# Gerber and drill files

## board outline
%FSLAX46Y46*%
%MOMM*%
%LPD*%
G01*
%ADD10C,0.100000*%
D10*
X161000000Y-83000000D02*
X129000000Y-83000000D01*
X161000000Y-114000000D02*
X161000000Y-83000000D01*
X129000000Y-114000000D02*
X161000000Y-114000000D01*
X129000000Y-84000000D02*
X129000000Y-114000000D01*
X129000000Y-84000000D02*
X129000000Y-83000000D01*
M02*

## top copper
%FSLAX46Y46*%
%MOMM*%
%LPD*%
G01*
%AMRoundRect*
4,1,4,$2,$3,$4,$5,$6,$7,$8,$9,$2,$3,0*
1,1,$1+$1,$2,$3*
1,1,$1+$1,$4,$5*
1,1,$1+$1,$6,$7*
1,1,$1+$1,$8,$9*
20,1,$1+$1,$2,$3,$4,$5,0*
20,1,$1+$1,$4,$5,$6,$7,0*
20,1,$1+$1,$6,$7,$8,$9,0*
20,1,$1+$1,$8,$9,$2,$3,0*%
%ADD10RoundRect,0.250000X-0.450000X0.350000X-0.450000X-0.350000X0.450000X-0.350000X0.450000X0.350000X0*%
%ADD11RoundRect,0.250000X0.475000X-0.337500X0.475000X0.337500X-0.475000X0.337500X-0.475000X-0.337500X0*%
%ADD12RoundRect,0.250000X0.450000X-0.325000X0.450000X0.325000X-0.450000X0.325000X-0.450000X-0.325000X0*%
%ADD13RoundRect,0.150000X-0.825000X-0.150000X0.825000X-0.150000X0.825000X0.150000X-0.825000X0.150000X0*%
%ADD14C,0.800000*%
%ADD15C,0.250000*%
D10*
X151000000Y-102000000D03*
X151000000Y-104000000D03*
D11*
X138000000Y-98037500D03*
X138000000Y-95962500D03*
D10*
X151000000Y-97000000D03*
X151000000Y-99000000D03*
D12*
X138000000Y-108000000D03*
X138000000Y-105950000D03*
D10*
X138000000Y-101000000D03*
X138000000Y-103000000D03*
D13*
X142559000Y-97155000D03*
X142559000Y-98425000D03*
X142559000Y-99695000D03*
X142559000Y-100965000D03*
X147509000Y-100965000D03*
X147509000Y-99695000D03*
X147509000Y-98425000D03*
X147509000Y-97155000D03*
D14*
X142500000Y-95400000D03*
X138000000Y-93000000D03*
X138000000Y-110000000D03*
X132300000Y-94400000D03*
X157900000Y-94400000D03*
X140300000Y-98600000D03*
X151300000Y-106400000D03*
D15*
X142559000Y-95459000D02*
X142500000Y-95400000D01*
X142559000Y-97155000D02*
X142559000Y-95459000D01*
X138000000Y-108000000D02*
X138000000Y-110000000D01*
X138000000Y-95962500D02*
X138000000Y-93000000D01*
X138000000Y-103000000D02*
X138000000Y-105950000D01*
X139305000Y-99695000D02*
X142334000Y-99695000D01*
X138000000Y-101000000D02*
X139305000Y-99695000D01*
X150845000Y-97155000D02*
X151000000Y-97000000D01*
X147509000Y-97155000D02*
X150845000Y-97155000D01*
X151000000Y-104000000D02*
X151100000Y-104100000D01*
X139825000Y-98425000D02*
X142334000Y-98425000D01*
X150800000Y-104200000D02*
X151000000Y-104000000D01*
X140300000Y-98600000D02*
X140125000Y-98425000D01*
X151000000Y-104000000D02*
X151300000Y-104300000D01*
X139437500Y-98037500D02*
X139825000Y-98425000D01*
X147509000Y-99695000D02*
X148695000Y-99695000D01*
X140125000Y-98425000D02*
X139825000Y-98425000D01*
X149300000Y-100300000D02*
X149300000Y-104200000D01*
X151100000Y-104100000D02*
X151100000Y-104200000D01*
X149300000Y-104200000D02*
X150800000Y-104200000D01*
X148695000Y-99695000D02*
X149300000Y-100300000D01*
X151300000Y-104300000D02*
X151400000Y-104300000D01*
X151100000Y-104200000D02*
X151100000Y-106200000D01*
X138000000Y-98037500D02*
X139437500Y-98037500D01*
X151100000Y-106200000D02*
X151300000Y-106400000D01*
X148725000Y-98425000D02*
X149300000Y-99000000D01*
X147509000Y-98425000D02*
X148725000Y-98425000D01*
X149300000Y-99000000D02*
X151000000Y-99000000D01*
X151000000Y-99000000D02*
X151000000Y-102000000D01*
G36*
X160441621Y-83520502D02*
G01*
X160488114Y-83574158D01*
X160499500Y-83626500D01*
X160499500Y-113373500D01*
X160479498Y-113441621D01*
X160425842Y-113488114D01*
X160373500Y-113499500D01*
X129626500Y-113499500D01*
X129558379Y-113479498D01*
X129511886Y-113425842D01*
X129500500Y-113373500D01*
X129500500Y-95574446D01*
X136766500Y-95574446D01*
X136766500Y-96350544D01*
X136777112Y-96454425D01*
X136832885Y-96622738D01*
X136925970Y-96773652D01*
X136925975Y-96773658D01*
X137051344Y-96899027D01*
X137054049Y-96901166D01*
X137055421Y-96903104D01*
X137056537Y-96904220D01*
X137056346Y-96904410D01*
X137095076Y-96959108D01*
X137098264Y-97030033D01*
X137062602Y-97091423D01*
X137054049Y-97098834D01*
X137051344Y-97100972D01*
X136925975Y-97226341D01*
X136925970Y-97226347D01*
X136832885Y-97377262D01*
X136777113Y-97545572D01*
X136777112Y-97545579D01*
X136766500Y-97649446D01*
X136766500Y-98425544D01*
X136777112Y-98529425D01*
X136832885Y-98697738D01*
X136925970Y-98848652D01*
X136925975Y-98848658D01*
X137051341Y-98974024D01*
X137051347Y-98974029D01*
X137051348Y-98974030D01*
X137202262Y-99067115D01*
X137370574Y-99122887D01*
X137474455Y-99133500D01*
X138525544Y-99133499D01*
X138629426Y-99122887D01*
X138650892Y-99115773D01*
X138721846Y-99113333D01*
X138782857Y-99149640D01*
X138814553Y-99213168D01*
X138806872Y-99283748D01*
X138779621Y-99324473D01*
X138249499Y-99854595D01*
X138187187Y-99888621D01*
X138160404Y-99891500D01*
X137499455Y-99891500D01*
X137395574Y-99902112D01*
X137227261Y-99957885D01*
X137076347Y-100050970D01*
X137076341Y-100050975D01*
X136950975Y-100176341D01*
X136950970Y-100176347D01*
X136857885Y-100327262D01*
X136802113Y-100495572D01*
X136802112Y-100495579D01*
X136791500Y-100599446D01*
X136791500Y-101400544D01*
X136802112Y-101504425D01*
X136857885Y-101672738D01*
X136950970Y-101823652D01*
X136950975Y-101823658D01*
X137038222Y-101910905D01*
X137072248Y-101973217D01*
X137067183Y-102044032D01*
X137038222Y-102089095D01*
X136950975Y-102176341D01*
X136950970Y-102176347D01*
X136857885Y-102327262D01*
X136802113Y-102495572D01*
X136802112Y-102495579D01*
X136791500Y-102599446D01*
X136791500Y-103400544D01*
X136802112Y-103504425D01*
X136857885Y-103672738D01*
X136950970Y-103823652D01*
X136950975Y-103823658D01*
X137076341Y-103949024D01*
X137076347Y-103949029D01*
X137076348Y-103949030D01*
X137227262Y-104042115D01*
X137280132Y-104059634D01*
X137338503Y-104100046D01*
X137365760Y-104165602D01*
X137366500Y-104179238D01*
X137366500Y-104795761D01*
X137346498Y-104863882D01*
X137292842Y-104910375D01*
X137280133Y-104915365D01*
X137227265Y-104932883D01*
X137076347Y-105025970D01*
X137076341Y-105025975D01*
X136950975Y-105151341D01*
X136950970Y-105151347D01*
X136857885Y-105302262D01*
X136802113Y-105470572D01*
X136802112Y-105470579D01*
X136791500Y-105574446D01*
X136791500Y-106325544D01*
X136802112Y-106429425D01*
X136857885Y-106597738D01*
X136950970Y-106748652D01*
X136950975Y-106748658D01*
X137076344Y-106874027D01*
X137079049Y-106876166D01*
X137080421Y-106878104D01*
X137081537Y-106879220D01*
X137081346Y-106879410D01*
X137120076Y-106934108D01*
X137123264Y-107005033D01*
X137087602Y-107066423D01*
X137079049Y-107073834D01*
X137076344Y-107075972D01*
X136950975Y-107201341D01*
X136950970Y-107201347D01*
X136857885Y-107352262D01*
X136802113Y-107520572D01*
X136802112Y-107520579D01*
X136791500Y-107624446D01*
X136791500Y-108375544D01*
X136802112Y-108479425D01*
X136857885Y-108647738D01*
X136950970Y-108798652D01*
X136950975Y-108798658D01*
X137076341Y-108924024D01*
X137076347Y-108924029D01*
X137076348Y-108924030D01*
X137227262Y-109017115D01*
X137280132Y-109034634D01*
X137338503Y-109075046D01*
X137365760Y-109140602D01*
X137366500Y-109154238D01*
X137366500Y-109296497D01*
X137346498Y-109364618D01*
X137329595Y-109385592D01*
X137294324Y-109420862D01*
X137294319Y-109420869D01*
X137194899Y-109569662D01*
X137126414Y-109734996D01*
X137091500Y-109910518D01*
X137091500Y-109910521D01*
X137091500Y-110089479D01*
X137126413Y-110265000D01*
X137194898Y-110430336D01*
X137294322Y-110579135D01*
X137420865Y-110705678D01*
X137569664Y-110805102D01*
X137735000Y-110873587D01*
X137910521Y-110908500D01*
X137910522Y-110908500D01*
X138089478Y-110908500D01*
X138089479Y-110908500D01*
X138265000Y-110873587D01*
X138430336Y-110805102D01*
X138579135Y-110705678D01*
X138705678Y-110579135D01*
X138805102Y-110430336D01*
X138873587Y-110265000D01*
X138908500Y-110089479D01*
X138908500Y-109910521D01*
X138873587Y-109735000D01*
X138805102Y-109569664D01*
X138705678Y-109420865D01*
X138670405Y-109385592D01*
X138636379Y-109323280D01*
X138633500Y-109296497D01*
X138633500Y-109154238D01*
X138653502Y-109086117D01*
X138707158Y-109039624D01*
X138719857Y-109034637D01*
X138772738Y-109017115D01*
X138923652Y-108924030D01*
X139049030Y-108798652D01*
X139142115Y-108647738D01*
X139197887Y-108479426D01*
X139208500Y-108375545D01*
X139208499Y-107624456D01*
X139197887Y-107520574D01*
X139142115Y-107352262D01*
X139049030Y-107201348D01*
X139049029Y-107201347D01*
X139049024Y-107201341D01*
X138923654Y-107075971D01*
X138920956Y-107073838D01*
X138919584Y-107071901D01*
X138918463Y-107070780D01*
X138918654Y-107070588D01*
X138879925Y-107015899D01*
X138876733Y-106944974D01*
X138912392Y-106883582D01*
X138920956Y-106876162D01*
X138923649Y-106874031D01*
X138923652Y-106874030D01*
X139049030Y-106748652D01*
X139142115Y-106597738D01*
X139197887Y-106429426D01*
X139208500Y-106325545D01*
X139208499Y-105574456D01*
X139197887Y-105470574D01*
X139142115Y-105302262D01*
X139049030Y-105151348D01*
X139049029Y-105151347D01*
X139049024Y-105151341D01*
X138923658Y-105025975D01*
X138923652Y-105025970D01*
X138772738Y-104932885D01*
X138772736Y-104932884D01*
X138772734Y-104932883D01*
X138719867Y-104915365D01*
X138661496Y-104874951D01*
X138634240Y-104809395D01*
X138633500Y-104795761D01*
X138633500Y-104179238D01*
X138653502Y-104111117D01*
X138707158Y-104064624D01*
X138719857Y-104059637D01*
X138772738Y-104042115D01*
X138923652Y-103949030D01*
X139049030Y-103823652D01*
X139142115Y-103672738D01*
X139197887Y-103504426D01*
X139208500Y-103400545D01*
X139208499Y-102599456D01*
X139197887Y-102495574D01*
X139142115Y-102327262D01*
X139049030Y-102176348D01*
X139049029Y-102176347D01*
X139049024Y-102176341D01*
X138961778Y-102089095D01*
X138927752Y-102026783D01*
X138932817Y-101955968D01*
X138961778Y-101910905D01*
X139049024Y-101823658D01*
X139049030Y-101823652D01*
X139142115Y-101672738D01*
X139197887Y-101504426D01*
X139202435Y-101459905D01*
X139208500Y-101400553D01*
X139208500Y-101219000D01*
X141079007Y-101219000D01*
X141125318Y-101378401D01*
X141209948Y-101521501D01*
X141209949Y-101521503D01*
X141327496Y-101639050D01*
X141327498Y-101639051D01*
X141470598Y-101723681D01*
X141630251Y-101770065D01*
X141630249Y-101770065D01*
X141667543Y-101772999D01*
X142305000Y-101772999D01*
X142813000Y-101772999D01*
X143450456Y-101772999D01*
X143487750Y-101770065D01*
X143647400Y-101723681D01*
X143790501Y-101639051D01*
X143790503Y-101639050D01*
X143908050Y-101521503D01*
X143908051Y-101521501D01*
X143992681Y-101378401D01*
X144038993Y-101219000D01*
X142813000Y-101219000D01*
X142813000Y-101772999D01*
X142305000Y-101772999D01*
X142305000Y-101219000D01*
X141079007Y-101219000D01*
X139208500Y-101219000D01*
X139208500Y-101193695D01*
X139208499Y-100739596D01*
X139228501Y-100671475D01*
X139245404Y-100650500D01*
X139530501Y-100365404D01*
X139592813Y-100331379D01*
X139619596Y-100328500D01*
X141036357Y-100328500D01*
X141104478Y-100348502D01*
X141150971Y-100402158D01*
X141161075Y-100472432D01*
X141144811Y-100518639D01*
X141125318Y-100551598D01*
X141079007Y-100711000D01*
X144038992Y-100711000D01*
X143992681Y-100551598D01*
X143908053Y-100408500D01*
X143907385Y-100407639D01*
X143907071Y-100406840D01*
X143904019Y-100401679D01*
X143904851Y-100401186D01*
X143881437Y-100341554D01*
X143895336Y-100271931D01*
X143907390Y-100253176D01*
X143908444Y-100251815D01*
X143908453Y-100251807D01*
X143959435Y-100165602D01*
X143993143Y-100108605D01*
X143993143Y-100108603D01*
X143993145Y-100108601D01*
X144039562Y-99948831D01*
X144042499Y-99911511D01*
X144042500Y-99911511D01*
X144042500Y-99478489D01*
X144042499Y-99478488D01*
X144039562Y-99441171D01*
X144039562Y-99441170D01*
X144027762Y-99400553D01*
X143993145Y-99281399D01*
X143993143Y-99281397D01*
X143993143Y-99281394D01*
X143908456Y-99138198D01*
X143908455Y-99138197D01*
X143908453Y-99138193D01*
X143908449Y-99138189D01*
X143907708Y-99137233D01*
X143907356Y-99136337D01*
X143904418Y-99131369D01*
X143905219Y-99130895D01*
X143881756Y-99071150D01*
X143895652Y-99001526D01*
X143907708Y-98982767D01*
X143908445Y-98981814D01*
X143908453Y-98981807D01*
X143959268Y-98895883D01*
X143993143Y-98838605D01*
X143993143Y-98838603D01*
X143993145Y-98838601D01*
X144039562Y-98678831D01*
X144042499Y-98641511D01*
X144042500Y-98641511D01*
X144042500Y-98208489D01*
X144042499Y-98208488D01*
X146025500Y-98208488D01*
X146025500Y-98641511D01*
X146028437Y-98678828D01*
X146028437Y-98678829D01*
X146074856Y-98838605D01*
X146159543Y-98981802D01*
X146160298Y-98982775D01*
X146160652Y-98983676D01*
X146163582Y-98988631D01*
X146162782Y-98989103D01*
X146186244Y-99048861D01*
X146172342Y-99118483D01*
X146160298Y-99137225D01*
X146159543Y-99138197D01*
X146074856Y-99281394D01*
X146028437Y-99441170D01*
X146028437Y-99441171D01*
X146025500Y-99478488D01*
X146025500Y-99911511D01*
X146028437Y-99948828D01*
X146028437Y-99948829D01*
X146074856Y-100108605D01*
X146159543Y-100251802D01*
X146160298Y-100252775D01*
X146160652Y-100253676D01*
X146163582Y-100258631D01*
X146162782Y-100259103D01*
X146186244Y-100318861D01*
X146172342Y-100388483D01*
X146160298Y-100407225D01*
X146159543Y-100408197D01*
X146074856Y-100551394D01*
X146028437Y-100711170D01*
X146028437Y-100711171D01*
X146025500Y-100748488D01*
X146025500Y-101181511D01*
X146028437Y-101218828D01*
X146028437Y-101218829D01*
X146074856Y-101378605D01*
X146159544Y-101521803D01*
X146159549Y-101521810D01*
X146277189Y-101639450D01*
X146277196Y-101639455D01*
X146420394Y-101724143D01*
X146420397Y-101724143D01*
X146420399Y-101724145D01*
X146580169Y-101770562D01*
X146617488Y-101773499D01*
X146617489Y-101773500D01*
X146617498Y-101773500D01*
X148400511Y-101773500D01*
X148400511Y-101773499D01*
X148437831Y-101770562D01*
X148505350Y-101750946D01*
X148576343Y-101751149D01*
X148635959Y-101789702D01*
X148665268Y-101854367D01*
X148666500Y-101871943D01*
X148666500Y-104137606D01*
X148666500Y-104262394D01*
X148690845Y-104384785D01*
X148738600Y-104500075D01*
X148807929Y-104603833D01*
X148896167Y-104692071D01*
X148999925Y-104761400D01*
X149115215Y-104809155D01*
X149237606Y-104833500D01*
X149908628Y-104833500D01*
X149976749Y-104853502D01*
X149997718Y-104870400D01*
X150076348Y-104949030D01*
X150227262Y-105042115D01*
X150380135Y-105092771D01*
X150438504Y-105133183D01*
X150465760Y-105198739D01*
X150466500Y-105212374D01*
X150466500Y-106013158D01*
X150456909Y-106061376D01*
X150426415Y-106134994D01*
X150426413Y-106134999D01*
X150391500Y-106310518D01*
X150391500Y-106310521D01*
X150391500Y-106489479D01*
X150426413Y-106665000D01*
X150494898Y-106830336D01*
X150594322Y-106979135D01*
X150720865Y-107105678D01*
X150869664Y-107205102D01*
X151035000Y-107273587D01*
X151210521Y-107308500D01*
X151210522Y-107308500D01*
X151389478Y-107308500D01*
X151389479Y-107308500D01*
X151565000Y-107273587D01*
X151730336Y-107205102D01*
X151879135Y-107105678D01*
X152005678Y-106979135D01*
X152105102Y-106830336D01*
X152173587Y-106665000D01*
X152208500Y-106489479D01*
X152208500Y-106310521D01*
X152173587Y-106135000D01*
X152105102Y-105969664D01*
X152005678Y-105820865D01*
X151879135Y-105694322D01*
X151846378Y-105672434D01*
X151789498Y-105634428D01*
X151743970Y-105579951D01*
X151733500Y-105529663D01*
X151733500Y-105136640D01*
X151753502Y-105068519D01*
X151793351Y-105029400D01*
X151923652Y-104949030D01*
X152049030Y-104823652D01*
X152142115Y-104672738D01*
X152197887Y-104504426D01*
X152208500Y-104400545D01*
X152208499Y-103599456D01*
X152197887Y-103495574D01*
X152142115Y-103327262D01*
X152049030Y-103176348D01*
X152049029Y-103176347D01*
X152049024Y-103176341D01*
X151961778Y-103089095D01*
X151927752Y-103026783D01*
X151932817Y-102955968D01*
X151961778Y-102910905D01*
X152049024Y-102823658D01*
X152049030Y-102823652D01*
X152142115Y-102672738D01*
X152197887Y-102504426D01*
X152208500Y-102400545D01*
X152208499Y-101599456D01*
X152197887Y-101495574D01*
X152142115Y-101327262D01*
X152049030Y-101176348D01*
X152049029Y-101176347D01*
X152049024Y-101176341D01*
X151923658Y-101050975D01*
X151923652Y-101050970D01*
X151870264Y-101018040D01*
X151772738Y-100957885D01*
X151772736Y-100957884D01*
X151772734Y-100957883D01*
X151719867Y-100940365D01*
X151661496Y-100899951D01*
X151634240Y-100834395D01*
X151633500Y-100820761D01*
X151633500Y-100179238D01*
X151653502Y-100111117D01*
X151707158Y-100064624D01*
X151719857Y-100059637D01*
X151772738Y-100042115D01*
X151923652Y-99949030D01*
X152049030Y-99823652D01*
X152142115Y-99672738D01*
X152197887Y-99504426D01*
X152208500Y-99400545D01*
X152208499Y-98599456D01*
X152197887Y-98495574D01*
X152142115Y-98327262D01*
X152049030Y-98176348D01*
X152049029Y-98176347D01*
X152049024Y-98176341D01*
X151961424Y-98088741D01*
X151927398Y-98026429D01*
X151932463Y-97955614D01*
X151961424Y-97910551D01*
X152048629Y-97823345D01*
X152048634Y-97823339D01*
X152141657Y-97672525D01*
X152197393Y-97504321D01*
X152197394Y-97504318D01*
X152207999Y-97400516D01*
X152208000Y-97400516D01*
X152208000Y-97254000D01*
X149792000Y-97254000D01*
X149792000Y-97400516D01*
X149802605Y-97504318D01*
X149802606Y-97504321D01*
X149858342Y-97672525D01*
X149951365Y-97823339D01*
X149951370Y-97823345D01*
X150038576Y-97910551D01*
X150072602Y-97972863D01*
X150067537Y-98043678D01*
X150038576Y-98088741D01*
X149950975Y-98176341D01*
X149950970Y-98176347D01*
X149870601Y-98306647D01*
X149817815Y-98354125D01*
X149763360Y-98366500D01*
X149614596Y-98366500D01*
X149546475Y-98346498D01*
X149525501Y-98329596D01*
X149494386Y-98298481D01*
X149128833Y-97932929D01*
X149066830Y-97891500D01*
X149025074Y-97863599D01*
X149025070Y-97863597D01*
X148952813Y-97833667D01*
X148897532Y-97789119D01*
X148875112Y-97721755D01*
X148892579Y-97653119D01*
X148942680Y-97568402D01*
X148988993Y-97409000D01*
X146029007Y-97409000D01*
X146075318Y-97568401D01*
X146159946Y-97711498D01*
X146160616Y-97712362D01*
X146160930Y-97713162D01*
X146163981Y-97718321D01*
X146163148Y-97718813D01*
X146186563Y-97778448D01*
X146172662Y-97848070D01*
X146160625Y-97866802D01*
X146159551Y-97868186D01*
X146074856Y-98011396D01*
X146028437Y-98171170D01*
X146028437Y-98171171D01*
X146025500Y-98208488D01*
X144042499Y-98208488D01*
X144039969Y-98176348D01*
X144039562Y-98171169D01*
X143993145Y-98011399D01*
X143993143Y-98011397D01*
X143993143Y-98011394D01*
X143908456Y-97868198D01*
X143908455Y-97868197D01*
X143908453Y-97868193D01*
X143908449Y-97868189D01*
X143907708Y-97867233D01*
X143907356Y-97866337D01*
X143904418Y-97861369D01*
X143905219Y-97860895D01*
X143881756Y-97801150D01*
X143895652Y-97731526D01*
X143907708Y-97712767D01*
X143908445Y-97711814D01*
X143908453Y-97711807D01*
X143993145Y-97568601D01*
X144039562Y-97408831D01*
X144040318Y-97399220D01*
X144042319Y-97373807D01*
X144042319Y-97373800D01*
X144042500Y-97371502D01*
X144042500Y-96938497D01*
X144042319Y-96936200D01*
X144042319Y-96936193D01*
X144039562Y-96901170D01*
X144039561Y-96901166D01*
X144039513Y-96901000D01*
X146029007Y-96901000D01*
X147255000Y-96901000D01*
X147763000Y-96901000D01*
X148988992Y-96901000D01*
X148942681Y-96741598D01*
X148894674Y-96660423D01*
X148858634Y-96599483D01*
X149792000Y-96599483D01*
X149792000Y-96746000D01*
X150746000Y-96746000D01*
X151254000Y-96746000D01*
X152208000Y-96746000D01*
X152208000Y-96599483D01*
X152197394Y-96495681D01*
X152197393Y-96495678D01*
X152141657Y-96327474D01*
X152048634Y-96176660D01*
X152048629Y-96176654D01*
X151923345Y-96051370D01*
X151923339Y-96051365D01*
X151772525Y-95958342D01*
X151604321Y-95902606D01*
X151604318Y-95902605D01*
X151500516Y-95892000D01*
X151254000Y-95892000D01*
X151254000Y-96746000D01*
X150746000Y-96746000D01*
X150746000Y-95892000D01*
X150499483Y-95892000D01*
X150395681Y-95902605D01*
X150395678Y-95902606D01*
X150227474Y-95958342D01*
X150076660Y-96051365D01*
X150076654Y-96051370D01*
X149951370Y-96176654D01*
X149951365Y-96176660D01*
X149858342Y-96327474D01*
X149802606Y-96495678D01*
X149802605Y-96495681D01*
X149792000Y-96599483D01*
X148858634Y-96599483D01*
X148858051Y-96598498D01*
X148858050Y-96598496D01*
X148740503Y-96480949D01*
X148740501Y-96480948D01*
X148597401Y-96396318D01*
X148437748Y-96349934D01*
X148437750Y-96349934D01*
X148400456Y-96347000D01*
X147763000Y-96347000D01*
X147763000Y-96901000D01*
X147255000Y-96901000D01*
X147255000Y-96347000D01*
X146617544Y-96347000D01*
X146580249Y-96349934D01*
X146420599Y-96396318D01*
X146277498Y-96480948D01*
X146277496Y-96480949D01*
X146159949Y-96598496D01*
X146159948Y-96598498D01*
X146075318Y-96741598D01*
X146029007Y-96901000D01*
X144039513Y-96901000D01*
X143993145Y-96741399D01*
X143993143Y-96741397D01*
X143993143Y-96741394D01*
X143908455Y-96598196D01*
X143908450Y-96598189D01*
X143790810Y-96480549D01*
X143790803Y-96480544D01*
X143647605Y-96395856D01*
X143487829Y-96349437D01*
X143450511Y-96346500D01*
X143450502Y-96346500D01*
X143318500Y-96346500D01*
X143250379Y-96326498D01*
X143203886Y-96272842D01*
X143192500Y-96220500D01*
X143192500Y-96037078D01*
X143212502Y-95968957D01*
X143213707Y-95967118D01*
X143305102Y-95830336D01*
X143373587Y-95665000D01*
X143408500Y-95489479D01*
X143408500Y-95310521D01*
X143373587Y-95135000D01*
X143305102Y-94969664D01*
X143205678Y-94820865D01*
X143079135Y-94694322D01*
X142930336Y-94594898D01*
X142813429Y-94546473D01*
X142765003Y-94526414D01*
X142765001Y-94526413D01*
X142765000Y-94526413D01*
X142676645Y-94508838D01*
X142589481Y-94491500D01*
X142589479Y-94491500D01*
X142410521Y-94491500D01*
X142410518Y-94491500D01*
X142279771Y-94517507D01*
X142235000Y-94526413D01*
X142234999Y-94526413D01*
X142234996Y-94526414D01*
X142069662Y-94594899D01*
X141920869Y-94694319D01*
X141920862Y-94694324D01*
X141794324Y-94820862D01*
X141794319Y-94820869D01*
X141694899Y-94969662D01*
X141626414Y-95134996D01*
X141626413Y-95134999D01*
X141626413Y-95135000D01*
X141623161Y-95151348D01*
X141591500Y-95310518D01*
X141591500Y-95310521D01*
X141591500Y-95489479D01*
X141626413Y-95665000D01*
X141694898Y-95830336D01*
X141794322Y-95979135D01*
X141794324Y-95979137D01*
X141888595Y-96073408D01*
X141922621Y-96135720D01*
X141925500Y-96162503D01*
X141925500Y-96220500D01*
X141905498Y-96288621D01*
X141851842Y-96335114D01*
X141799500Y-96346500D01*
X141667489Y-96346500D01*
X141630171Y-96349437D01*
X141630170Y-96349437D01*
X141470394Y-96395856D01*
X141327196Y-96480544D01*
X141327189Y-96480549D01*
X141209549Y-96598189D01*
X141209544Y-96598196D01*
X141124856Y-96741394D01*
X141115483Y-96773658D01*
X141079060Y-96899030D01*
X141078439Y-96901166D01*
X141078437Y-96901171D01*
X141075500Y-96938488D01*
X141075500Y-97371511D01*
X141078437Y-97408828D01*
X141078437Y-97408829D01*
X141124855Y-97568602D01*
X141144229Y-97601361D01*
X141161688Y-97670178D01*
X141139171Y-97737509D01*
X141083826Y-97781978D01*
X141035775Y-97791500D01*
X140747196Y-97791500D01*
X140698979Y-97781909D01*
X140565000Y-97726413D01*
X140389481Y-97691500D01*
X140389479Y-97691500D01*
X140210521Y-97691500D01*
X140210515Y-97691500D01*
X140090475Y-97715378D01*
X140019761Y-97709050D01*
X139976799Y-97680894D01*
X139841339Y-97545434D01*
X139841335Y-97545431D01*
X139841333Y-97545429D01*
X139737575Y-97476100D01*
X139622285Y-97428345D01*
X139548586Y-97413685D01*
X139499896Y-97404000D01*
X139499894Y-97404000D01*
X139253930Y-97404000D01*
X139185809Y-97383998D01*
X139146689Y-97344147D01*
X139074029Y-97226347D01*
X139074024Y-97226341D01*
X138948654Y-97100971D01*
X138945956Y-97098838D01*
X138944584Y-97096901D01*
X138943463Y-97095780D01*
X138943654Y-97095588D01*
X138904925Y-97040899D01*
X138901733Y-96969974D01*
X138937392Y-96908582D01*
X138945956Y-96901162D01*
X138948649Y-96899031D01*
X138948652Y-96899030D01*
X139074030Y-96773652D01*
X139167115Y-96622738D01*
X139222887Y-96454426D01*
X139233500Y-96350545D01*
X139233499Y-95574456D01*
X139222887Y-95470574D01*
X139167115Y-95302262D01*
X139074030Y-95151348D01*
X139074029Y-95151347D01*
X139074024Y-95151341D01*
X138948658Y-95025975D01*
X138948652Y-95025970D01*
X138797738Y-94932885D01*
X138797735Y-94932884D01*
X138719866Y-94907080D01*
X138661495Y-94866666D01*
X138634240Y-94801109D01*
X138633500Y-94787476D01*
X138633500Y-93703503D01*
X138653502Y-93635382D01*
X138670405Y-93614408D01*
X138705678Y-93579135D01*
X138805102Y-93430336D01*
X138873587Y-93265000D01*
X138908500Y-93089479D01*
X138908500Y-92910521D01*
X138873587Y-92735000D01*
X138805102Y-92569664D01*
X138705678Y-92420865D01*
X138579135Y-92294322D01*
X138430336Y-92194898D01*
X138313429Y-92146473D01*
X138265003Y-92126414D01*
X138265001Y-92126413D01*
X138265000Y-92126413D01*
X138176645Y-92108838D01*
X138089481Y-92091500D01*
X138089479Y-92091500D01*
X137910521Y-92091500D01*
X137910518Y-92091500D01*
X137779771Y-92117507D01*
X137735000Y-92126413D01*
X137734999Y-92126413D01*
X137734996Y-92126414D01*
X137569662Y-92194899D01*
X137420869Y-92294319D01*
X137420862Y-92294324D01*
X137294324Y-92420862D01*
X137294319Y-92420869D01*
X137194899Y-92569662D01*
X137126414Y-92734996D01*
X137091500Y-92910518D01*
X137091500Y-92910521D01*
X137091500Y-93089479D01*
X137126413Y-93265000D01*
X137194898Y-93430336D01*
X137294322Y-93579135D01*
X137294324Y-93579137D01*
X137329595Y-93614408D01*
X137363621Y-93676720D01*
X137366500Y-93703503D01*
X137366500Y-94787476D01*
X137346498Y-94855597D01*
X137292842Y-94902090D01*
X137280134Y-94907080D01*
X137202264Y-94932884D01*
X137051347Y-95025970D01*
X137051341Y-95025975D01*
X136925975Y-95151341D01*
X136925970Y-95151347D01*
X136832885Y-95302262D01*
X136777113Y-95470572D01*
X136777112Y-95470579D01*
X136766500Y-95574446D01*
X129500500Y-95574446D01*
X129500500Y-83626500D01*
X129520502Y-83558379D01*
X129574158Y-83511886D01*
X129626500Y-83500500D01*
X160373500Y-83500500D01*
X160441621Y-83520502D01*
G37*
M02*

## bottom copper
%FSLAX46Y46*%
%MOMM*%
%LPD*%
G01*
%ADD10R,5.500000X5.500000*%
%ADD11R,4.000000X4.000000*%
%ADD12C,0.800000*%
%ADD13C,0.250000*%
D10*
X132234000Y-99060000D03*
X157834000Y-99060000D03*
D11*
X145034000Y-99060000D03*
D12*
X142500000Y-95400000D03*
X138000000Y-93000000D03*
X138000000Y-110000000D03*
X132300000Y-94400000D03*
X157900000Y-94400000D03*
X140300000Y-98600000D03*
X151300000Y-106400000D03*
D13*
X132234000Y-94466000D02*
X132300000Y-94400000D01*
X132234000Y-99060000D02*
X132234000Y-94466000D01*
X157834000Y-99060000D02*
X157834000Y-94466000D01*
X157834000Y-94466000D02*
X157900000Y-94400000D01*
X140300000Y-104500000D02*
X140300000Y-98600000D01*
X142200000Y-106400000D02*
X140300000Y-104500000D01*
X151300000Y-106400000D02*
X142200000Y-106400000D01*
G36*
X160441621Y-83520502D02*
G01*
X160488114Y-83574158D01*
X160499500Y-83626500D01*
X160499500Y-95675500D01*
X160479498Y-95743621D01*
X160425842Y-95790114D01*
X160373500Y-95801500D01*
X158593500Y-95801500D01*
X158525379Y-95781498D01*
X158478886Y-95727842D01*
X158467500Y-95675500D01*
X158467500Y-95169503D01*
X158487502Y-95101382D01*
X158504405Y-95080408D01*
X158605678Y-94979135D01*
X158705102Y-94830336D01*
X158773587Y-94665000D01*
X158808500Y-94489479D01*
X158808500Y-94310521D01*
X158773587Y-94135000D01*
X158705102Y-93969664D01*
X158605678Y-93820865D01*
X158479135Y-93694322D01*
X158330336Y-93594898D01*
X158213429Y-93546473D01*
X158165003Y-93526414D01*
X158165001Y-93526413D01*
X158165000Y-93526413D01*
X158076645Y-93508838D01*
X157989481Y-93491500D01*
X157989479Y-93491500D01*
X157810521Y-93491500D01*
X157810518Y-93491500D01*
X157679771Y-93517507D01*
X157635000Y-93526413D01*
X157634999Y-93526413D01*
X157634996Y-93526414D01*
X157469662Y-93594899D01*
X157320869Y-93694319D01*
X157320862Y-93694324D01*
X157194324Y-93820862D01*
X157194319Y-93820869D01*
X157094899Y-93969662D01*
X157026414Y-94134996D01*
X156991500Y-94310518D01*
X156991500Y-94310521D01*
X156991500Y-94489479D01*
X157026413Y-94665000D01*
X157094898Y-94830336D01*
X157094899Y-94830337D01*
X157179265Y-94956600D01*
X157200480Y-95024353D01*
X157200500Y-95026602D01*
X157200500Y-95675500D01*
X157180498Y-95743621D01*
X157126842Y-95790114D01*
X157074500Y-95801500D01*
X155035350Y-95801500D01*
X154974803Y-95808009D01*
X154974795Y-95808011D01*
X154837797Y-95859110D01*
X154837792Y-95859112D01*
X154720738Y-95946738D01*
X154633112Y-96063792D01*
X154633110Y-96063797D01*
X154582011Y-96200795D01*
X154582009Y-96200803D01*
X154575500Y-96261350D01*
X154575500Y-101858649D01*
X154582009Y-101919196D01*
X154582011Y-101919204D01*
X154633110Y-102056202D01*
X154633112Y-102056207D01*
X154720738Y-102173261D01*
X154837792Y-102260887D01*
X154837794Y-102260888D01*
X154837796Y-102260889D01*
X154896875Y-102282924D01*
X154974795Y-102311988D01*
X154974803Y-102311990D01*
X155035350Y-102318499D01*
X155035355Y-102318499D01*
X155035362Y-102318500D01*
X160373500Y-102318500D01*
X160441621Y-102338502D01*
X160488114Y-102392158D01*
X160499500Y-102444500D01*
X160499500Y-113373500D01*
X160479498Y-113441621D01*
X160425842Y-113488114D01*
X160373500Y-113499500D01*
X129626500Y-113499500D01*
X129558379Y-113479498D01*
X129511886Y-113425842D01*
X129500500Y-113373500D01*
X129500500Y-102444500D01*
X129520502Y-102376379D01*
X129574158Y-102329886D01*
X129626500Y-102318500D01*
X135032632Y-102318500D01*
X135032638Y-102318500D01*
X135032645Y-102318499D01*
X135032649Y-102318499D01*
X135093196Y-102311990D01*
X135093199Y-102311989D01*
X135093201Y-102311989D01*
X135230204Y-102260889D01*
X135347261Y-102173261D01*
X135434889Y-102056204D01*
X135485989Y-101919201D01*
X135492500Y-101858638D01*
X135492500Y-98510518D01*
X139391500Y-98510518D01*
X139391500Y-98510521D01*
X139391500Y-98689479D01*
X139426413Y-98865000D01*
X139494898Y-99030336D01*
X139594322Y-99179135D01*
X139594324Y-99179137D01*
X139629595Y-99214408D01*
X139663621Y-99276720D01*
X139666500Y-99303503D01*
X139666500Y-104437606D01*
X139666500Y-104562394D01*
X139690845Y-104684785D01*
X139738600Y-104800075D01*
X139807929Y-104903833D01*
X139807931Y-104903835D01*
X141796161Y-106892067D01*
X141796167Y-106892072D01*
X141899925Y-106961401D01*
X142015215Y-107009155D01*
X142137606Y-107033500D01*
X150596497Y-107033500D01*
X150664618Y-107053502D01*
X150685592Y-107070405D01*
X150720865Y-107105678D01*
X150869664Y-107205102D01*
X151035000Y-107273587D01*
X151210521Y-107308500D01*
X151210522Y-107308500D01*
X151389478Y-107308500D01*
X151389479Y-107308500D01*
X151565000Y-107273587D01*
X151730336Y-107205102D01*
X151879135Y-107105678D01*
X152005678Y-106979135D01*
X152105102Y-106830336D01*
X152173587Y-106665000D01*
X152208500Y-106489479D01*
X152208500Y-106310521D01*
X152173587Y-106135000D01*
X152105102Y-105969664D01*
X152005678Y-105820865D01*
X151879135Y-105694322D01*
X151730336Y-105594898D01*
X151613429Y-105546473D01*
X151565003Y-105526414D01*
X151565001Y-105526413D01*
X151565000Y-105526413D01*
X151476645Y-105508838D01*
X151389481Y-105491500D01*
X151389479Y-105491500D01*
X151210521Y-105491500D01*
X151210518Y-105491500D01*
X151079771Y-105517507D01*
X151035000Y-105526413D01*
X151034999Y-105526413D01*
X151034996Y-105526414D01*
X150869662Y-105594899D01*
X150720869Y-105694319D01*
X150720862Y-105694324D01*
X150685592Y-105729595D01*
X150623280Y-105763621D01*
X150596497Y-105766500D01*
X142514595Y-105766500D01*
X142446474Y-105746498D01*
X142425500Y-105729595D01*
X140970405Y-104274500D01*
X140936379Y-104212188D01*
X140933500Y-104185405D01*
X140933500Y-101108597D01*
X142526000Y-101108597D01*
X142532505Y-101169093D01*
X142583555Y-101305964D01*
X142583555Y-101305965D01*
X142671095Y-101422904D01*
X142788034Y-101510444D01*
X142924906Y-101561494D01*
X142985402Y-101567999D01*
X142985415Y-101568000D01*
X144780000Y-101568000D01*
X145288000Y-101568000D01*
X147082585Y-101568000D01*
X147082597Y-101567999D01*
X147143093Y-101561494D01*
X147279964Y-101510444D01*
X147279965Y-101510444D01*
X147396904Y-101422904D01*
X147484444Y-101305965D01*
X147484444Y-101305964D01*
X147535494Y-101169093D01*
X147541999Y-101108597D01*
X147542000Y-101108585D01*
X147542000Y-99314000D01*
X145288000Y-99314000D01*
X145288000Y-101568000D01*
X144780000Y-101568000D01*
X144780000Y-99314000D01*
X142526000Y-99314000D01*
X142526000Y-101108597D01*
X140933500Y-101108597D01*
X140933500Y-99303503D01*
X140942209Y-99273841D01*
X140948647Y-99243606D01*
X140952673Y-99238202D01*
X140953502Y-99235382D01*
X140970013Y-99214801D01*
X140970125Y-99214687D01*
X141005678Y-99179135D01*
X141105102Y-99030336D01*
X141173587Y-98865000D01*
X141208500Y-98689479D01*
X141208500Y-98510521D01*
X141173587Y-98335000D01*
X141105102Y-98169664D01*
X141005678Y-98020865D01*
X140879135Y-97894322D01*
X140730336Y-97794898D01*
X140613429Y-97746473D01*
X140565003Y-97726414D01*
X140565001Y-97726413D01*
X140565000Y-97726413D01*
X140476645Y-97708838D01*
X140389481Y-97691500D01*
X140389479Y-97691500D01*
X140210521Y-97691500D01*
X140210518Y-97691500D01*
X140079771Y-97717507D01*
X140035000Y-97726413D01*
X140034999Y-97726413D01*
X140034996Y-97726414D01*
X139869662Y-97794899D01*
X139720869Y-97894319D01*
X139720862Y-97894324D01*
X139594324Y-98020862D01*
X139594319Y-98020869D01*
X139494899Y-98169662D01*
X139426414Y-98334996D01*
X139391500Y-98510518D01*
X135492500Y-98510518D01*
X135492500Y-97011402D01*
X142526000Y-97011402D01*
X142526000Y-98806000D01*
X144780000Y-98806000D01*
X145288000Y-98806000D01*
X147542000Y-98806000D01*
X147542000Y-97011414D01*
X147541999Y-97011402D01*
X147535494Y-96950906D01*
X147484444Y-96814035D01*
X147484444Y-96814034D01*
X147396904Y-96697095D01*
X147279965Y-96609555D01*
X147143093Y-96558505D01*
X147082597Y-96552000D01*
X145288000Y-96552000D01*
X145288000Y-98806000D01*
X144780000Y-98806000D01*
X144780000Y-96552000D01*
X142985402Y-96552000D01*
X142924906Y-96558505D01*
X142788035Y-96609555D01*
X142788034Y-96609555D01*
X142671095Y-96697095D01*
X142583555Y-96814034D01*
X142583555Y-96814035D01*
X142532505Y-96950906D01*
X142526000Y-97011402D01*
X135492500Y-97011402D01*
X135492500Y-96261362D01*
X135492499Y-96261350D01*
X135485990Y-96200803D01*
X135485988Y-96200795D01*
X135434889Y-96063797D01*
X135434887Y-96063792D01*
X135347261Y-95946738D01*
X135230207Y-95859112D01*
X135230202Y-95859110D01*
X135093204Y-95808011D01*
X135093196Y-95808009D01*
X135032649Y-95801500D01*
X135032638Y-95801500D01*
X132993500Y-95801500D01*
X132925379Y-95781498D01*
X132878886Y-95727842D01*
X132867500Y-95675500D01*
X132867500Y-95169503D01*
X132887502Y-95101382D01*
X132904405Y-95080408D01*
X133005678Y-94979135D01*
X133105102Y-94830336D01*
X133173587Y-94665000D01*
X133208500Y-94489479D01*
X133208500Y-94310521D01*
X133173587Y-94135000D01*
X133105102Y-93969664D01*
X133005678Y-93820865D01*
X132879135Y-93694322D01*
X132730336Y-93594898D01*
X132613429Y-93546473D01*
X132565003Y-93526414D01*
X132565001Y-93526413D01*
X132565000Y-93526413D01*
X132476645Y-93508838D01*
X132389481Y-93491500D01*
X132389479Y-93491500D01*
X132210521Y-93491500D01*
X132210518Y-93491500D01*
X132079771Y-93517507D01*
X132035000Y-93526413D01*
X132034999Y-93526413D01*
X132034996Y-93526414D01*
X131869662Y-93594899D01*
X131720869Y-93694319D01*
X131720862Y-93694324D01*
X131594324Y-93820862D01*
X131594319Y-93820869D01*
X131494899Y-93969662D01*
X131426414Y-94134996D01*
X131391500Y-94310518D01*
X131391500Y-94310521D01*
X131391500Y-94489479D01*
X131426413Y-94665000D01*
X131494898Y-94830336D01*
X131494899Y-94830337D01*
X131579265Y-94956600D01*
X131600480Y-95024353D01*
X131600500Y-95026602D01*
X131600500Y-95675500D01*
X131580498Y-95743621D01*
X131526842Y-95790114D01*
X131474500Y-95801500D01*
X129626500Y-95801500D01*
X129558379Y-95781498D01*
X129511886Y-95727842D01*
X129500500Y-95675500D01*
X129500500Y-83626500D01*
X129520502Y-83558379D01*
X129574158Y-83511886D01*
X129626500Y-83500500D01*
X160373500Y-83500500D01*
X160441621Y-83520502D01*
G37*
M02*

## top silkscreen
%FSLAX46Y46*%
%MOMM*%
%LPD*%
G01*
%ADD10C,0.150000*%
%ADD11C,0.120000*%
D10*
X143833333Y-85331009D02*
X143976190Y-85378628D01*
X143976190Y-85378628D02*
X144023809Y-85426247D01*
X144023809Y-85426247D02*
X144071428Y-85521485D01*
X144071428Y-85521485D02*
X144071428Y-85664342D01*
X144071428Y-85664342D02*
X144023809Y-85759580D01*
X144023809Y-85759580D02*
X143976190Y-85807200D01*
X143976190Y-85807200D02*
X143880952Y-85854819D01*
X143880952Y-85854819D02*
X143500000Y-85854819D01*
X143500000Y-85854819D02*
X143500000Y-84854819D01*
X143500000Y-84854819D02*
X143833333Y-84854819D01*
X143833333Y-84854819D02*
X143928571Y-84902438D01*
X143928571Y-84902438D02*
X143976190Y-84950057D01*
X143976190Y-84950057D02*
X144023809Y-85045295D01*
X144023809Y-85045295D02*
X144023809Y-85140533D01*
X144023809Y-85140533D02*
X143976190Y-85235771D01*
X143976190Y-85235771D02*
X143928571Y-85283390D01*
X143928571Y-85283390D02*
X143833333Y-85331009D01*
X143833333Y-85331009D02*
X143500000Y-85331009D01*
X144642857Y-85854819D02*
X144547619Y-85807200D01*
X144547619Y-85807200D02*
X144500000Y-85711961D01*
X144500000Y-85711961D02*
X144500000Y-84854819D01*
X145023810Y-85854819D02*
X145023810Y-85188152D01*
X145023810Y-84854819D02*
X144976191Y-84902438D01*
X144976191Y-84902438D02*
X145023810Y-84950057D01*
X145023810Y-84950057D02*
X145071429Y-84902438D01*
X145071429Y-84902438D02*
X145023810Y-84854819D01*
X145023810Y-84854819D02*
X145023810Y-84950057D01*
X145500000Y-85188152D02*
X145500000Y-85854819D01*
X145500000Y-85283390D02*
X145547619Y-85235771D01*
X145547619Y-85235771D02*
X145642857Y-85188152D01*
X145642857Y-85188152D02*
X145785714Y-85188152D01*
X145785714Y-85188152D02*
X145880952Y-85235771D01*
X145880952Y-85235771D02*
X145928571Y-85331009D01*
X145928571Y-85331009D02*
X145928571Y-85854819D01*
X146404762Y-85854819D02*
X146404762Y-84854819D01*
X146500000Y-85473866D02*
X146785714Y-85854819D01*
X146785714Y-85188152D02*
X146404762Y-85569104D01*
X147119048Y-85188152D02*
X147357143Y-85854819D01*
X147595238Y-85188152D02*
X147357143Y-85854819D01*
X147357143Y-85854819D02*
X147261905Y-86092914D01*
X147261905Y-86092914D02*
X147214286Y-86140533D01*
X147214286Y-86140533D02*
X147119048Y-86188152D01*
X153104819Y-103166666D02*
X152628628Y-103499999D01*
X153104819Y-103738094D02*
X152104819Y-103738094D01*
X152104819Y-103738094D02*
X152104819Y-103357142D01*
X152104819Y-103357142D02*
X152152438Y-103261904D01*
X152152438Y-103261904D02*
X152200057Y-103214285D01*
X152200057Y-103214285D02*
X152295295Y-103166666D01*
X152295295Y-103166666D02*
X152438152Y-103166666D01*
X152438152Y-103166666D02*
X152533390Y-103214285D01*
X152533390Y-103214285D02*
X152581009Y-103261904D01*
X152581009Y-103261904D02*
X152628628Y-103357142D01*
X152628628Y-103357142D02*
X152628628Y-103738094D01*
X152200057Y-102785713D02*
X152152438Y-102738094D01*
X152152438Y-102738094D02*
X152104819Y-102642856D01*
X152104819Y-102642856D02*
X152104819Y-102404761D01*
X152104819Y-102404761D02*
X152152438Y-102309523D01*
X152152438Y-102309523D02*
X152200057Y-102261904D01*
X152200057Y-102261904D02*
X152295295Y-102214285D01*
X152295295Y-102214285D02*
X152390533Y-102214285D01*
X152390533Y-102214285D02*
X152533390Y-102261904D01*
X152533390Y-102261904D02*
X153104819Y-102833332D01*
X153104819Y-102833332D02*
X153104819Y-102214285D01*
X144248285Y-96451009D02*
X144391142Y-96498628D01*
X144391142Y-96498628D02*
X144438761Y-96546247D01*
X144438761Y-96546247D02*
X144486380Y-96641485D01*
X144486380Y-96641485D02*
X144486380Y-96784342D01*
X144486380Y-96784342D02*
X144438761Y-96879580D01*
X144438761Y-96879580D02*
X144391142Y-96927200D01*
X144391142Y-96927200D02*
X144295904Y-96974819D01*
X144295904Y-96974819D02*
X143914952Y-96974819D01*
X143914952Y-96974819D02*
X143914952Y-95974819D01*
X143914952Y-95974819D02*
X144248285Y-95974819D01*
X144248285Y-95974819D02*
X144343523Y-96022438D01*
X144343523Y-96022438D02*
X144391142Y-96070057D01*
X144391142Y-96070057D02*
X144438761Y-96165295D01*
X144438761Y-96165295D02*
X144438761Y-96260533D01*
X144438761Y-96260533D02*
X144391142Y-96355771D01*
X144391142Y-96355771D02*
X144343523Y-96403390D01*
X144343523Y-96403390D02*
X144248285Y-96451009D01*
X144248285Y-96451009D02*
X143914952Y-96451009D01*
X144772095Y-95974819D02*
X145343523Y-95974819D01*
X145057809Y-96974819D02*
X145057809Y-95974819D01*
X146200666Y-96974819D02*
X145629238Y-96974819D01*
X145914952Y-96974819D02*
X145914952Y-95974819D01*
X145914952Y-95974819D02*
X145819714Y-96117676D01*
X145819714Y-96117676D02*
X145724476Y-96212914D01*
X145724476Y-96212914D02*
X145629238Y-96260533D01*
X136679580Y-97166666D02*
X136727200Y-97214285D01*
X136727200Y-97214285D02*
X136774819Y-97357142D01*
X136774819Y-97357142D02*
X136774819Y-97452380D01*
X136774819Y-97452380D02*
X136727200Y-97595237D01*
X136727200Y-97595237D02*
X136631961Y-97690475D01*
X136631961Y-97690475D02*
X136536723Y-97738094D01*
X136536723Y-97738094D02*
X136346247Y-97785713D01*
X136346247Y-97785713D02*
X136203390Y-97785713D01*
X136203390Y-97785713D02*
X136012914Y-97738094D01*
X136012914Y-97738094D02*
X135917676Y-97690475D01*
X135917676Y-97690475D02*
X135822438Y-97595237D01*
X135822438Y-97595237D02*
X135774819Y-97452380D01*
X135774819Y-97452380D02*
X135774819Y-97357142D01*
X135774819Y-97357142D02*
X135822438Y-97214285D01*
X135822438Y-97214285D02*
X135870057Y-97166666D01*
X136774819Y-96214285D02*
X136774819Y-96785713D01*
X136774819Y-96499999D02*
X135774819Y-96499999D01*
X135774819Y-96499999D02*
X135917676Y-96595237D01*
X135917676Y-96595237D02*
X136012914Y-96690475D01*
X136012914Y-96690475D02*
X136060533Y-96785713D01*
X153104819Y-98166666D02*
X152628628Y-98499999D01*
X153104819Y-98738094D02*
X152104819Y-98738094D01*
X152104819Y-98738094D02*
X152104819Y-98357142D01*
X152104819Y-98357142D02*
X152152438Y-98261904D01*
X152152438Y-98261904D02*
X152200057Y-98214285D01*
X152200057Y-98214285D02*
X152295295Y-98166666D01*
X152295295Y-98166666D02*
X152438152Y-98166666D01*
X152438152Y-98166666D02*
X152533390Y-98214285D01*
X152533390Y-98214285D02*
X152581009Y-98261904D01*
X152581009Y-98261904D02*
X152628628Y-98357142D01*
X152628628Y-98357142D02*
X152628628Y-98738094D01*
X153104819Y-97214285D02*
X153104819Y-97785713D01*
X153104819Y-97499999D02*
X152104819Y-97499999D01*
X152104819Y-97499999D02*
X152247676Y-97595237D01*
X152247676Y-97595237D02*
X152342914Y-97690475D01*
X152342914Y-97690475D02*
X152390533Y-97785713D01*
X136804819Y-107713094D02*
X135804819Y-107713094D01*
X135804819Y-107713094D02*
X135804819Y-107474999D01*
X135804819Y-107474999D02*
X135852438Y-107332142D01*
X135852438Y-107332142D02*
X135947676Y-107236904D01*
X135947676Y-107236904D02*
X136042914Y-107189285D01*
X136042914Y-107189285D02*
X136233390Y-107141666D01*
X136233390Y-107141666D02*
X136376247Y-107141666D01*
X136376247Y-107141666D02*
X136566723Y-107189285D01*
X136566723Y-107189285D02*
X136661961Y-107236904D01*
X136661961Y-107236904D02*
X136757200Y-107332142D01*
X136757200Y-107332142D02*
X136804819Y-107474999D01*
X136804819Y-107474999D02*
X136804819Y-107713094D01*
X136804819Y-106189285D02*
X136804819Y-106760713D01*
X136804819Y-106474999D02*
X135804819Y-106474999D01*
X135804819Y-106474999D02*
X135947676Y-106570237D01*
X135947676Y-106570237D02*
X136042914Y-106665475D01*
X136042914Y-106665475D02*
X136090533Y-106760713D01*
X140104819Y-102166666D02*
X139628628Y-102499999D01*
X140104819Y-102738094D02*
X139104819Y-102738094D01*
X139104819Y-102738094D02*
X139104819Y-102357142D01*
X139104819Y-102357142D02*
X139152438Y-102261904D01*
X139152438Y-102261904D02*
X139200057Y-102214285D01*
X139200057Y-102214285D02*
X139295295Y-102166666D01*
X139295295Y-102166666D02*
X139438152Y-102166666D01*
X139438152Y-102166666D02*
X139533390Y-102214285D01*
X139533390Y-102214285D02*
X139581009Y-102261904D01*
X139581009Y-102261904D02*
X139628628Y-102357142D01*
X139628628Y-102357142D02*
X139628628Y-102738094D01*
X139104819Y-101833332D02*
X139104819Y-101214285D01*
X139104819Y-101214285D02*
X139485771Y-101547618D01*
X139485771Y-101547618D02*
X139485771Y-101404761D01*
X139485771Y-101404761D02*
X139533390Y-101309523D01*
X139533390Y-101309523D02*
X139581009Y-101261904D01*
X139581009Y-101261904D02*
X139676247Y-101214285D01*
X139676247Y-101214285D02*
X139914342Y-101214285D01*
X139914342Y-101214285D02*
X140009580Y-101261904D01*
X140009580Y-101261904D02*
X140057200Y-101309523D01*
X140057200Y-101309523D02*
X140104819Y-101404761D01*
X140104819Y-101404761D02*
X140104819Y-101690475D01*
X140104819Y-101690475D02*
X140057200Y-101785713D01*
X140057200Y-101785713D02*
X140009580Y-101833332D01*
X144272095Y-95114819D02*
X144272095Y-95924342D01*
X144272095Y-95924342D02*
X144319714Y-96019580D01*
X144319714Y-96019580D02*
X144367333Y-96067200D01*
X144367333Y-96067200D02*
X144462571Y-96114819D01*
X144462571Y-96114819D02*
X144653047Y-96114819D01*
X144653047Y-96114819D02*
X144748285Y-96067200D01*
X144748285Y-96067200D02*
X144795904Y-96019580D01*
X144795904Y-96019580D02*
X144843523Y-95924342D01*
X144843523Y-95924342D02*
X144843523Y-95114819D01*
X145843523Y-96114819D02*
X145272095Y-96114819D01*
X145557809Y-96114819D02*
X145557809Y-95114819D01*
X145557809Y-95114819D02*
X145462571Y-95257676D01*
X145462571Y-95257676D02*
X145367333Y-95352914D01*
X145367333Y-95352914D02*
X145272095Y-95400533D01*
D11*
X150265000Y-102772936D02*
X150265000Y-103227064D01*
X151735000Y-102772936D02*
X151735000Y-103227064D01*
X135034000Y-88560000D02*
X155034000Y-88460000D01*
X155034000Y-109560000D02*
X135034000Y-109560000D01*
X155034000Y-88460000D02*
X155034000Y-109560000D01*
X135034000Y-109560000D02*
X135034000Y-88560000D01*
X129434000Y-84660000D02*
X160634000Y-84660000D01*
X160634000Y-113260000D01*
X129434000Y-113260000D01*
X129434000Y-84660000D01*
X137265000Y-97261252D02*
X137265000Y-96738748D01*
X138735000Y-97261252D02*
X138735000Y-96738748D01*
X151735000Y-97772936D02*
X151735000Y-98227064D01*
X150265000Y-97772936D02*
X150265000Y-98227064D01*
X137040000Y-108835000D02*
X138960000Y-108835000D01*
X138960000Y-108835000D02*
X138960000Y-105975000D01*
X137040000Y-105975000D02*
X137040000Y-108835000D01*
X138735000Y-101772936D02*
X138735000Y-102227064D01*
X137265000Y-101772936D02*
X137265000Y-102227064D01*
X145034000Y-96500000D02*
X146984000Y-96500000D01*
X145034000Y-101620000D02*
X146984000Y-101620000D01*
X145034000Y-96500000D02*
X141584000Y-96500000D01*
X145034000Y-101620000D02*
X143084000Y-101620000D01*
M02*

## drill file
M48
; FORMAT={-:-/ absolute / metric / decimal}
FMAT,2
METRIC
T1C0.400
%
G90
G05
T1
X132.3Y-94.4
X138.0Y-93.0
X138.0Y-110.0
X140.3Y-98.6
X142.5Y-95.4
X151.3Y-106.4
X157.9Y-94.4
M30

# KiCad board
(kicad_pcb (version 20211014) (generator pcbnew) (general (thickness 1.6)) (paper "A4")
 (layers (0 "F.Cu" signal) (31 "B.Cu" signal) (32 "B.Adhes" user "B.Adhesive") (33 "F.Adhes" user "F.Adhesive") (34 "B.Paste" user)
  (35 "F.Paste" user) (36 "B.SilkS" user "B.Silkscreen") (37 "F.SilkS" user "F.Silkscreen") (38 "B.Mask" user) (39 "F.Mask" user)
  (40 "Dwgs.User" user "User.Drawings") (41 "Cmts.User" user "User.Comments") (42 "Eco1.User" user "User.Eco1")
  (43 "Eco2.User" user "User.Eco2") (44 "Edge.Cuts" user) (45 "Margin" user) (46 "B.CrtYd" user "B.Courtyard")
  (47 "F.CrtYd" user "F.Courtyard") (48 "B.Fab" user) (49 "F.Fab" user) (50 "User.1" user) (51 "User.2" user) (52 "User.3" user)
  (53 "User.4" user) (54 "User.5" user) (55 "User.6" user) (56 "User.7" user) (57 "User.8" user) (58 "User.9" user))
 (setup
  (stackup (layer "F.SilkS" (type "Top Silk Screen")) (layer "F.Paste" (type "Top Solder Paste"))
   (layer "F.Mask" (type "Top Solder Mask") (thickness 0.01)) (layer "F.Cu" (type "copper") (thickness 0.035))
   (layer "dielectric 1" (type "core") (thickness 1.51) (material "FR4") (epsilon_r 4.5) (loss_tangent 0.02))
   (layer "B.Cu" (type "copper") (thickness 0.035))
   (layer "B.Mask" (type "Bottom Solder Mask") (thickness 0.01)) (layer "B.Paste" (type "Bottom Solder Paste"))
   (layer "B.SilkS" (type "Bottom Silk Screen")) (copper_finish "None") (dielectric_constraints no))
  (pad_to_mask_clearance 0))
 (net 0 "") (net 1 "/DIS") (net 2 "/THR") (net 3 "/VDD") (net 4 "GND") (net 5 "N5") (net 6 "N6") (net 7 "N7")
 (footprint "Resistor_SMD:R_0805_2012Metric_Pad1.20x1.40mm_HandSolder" (layer "F.Cu") (at 151 103 -90)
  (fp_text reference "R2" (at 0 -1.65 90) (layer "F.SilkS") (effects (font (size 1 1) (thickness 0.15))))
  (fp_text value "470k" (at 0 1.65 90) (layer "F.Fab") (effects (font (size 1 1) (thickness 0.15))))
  (fp_line (start -0.227064 0.735) (end 0.227064 0.735) (layer "F.SilkS") (width 0.12))
  (fp_line (start -0.227064 -0.735) (end 0.227064 -0.735) (layer "F.SilkS") (width 0.12))
  (pad "1" smd roundrect (at -1 0 270) (size 1.2 1.4) (layers "F.Cu" "F.Paste" "F.Mask") (roundrect_rratio 0.2083333333) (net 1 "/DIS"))
  (pad "2" smd roundrect (at 1 0 270) (size 1.2 1.4) (layers "F.Cu" "F.Paste" "F.Mask") (roundrect_rratio 0.2083333333) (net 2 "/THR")))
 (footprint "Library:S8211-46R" (layer "F.Cu") (at 145.034 99.06)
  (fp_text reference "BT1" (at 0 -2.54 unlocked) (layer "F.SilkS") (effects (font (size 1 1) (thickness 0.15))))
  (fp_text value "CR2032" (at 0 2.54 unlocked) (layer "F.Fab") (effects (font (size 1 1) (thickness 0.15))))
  (fp_line (start -10 -10.5) (end 10 -10.6) (layer "F.SilkS") (width 0.12))
  (fp_line (start 10 10.5) (end -10 10.5) (layer "F.SilkS") (width 0.12))
  (fp_line (start 10 -10.6) (end 10 10.5) (layer "F.SilkS") (width 0.12))
  (fp_line (start -10 10.5) (end -10 -10.5) (layer "F.SilkS") (width 0.12))
  (fp_rect (start -15.6 14.2) (end 15.6 -14.4) (layer "F.SilkS") (width 0.12) (fill none))
  (pad "1" smd rect (at -12.8 0) (size 5.5 5.5) (layers "B.Cu" "F.Paste" "F.Mask") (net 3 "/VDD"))
  (pad "1" smd rect (at 12.8 0) (size 5.5 5.5) (layers "B.Cu" "F.Paste" "F.Mask") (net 3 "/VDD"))
  (pad "2" smd rect (at 0 0) (size 4 4) (layers "B.Cu" "F.Paste" "F.Mask") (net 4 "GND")))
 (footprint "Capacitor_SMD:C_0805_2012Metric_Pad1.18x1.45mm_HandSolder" (layer "F.Cu") (at 138 97 90)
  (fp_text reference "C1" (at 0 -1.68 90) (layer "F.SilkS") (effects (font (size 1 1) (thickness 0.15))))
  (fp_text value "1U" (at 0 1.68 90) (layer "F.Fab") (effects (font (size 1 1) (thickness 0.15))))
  (fp_line (start -0.261252 -0.735) (end 0.261252 -0.735) (layer "F.SilkS") (width 0.12))
  (fp_line (start -0.261252 0.735) (end 0.261252 0.735) (layer "F.SilkS") (width 0.12))
  (pad "1" smd roundrect (at -1.0375 0 90) (size 1.175 1.45) (layers "F.Cu" "F.Paste" "F.Mask") (roundrect_rratio 0.2127659574)
   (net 2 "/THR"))
  (pad "2" smd roundrect (at 1.0375 0 90) (size 1.175 1.45) (layers "F.Cu" "F.Paste" "F.Mask") (roundrect_rratio 0.2127659574) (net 4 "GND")))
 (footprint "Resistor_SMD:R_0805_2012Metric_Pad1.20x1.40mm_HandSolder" (layer "F.Cu") (at 151 98 -90)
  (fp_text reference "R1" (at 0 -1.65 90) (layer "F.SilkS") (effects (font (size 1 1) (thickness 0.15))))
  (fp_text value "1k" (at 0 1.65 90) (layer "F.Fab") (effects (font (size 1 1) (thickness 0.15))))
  (fp_line (start -0.227064 -0.735) (end 0.227064 -0.735) (layer "F.SilkS") (width 0.12))
  (fp_line (start -0.227064 0.735) (end 0.227064 0.735) (layer "F.SilkS") (width 0.12))
  (pad "1" smd roundrect (at -1 0 270) (size 1.2 1.4) (layers "F.Cu" "F.Paste" "F.Mask") (roundrect_rratio 0.2083333333) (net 3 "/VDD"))
  (pad "2" smd roundrect (at 1 0 270) (size 1.2 1.4) (layers "F.Cu" "F.Paste" "F.Mask") (roundrect_rratio 0.2083333333) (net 1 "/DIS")))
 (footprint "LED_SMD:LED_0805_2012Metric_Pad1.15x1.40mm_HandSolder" (layer "F.Cu") (at 138 106.975 90)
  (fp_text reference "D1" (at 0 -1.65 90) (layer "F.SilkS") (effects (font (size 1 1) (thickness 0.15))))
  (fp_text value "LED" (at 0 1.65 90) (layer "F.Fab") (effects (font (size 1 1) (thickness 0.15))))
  (fp_line (start -1.86 -0.96) (end -1.86 0.96) (layer "F.SilkS") (width 0.12))
  (fp_line (start -1.86 0.96) (end 1 0.96) (layer "F.SilkS") (width 0.12))
  (fp_line (start 1 -0.96) (end -1.86 -0.96) (layer "F.SilkS") (width 0.12))
  (pad "1" smd roundrect (at -1.025 0 90) (size 1.15 1.4) (layers "F.Cu" "F.Paste" "F.Mask") (roundrect_rratio 0.2173913043) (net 4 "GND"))
  (pad "2" smd roundrect (at 1.025 0 90) (size 1.15 1.4) (layers "F.Cu" "F.Paste" "F.Mask") (roundrect_rratio 0.2173913043) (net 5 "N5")))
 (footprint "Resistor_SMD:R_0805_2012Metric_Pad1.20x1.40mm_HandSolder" (layer "F.Cu") (at 138 102 -90)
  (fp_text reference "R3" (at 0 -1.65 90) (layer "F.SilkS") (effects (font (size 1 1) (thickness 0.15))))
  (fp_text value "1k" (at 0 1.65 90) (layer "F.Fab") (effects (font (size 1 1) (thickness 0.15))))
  (fp_line (start -0.227064 -0.735) (end 0.227064 -0.735) (layer "F.SilkS") (width 0.12))
  (fp_line (start -0.227064 0.735) (end 0.227064 0.735) (layer "F.SilkS") (width 0.12))
  (pad "1" smd roundrect (at -1 0 270) (size 1.2 1.4) (layers "F.Cu" "F.Paste" "F.Mask") (roundrect_rratio 0.2083333333) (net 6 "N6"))
  (pad "2" smd roundrect (at 1 0 270) (size 1.2 1.4) (layers "F.Cu" "F.Paste" "F.Mask") (roundrect_rratio 0.2083333333) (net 5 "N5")))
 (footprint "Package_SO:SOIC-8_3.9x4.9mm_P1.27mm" (layer "F.Cu") (at 145.034 99.06)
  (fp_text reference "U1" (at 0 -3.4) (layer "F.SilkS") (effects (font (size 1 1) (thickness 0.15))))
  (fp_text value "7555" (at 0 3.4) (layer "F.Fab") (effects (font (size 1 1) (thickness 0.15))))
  (fp_line (start 0 -2.56) (end 1.95 -2.56) (layer "F.SilkS") (width 0.12))
  (fp_line (start 0 2.56) (end 1.95 2.56) (layer "F.SilkS") (width 0.12))
  (fp_line (start 0 -2.56) (end -3.45 -2.56) (layer "F.SilkS") (width 0.12))
  (fp_line (start 0 2.56) (end -1.95 2.56) (layer "F.SilkS") (width 0.12))
  (pad "1" smd roundrect (at -2.475 -1.905) (size 1.95 0.6) (layers "F.Cu" "F.Paste" "F.Mask") (roundrect_rratio 0.25) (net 4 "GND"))
  (pad "2" smd roundrect (at -2.475 -0.635) (size 1.95 0.6) (layers "F.Cu" "F.Paste" "F.Mask") (roundrect_rratio 0.25) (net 2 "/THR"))
  (pad "3" smd roundrect (at -2.475 0.635) (size 1.95 0.6) (layers "F.Cu" "F.Paste" "F.Mask") (roundrect_rratio 0.25) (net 6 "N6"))
  (pad "4" smd roundrect (at -2.475 1.905) (size 1.95 0.6) (layers "F.Cu" "F.Paste" "F.Mask") (roundrect_rratio 0.25) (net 3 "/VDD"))
  (pad "5" smd roundrect (at 2.475 1.905) (size 1.95 0.6) (layers "F.Cu" "F.Paste" "F.Mask") (roundrect_rratio 0.25) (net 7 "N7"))
  (pad "6" smd roundrect (at 2.475 0.635) (size 1.95 0.6) (layers "F.Cu" "F.Paste" "F.Mask") (roundrect_rratio 0.25) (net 2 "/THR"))
  (pad "7" smd roundrect (at 2.475 -0.635) (size 1.95 0.6) (layers "F.Cu" "F.Paste" "F.Mask") (roundrect_rratio 0.25) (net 1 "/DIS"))
  (pad "8" smd roundrect (at 2.475 -1.905) (size 1.95 0.6) (layers "F.Cu" "F.Paste" "F.Mask") (roundrect_rratio 0.25) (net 3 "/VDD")))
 (gr_line (start 161 83) (end 129 83) (layer "Edge.Cuts") (width 0.1))
 (gr_line (start 161 114) (end 161 83) (layer "Edge.Cuts") (width 0.1))
 (gr_line (start 129 114) (end 161 114) (layer "Edge.Cuts") (width 0.1))
 (gr_line (start 129 84) (end 129 114) (layer "Edge.Cuts") (width 0.1))
 (gr_line (start 129 84) (end 129 83) (layer "Edge.Cuts") (width 0.1))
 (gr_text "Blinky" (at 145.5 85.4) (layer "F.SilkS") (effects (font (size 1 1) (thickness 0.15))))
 (segment (start 142.559 95.459) (end 142.5 95.4) (width 0.25) (layer "F.Cu") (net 4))
 (segment (start 142.559 97.155) (end 142.559 95.459) (width 0.25) (layer "F.Cu") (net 4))
 (segment (start 138 108) (end 138 110) (width 0.25) (layer "F.Cu") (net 4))
 (segment (start 138 95.9625) (end 138 93) (width 0.25) (layer "F.Cu") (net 4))
 (via (at 142.5 95.4) (size 0.8) (drill 0.4) (layers "F.Cu" "B.Cu") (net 4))
 (via (at 138 93) (size 0.8) (drill 0.4) (layers "F.Cu" "B.Cu") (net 4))
 (via (at 138 110) (size 0.8) (drill 0.4) (layers "F.Cu" "B.Cu") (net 4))
 (segment (start 138 103) (end 138 105.95) (width 0.25) (layer "F.Cu") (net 5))
 (segment (start 139.305 99.695) (end 142.334 99.695) (width 0.25) (layer "F.Cu") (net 6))
 (segment (start 138 101) (end 139.305 99.695) (width 0.25) (layer "F.Cu") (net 6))
 (segment (start 150.845 97.155) (end 151 97) (width 0.25) (layer "F.Cu") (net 3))
 (segment (start 147.509 97.155) (end 150.845 97.155) (width 0.25) (layer "F.Cu") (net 3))
 (via (at 132.3 94.4) (size 0.8) (drill 0.4) (layers "F.Cu" "B.Cu") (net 3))
 (via (at 157.9 94.4) (size 0.8) (drill 0.4) (layers "F.Cu" "B.Cu") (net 3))
 (segment (start 132.234 94.466) (end 132.3 94.4) (width 0.25) (layer "B.Cu") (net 3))
 (segment (start 132.234 99.06) (end 132.234 94.466) (width 0.25) (layer "B.Cu") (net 3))
 (segment (start 157.834 99.06) (end 157.834 94.466) (width 0.25) (layer "B.Cu") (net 3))
 (segment (start 157.834 94.466) (end 157.9 94.4) (width 0.25) (layer "B.Cu") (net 3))
 (segment (start 151 104) (end 151.1 104.1) (width 0.25) (layer "F.Cu") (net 2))
 (segment (start 139.825 98.425) (end 142.334 98.425) (width 0.25) (layer "F.Cu") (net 2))
 (segment (start 150.8 104.2) (end 151 104) (width 0.25) (layer "F.Cu") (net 2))
 (segment (start 140.3 98.6) (end 140.125 98.425) (width 0.25) (layer "F.Cu") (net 2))
 (segment (start 151 104) (end 151.3 104.3) (width 0.25) (layer "F.Cu") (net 2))
 (segment (start 139.4375 98.0375) (end 139.825 98.425) (width 0.25) (layer "F.Cu") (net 2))
 (segment (start 147.509 99.695) (end 148.695 99.695) (width 0.25) (layer "F.Cu") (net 2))
 (segment (start 140.125 98.425) (end 139.825 98.425) (width 0.25) (layer "F.Cu") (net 2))
 (segment (start 149.3 100.3) (end 149.3 104.2) (width 0.25) (layer "F.Cu") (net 2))
 (segment (start 151.1 104.1) (end 151.1 104.2) (width 0.25) (layer "F.Cu") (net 2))
 (segment (start 149.3 104.2) (end 150.8 104.2) (width 0.25) (layer "F.Cu") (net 2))
 (segment (start 148.695 99.695) (end 149.3 100.3) (width 0.25) (layer "F.Cu") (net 2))
 (segment (start 151.3 104.3) (end 151.4 104.3) (width 0.25) (layer "F.Cu") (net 2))
 (segment (start 151.1 104.2) (end 151.1 106.2) (width 0.25) (layer "F.Cu") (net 2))
 (segment (start 138 98.0375) (end 139.4375 98.0375) (width 0.25) (layer "F.Cu") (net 2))
 (segment (start 151.1 106.2) (end 151.3 106.4) (width 0.25) (layer "F.Cu") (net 2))
 (via (at 140.3 98.6) (size 0.8) (drill 0.4) (layers "F.Cu" "B.Cu") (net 2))
 (via (at 151.3 106.4) (size 0.8) (drill 0.4) (layers "F.Cu" "B.Cu") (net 2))
 (segment (start 140.3 104.5) (end 140.3 98.6) (width 0.25) (layer "B.Cu") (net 2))
 (segment (start 142.2 106.4) (end 140.3 104.5) (width 0.25) (layer "B.Cu") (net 2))
 (segment (start 151.3 106.4) (end 142.2 106.4) (width 0.25) (layer "B.Cu") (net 2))
 (segment (start 148.725 98.425) (end 149.3 99) (width 0.25) (layer "F.Cu") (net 1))
 (segment (start 147.509 98.425) (end 148.725 98.425) (width 0.25) (layer "F.Cu") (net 1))
 (segment (start 149.3 99) (end 151 99) (width 0.25) (layer "F.Cu") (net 1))
 (segment (start 151 99) (end 151 102) (width 0.25) (layer "F.Cu") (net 1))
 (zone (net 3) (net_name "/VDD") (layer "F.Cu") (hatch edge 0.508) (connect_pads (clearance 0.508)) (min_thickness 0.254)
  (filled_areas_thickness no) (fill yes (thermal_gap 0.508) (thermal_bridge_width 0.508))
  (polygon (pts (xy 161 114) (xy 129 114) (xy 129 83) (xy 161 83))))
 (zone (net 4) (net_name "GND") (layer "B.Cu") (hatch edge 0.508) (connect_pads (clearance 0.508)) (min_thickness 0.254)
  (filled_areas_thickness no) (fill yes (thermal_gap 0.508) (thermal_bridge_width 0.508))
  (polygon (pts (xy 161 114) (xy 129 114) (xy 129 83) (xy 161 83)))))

